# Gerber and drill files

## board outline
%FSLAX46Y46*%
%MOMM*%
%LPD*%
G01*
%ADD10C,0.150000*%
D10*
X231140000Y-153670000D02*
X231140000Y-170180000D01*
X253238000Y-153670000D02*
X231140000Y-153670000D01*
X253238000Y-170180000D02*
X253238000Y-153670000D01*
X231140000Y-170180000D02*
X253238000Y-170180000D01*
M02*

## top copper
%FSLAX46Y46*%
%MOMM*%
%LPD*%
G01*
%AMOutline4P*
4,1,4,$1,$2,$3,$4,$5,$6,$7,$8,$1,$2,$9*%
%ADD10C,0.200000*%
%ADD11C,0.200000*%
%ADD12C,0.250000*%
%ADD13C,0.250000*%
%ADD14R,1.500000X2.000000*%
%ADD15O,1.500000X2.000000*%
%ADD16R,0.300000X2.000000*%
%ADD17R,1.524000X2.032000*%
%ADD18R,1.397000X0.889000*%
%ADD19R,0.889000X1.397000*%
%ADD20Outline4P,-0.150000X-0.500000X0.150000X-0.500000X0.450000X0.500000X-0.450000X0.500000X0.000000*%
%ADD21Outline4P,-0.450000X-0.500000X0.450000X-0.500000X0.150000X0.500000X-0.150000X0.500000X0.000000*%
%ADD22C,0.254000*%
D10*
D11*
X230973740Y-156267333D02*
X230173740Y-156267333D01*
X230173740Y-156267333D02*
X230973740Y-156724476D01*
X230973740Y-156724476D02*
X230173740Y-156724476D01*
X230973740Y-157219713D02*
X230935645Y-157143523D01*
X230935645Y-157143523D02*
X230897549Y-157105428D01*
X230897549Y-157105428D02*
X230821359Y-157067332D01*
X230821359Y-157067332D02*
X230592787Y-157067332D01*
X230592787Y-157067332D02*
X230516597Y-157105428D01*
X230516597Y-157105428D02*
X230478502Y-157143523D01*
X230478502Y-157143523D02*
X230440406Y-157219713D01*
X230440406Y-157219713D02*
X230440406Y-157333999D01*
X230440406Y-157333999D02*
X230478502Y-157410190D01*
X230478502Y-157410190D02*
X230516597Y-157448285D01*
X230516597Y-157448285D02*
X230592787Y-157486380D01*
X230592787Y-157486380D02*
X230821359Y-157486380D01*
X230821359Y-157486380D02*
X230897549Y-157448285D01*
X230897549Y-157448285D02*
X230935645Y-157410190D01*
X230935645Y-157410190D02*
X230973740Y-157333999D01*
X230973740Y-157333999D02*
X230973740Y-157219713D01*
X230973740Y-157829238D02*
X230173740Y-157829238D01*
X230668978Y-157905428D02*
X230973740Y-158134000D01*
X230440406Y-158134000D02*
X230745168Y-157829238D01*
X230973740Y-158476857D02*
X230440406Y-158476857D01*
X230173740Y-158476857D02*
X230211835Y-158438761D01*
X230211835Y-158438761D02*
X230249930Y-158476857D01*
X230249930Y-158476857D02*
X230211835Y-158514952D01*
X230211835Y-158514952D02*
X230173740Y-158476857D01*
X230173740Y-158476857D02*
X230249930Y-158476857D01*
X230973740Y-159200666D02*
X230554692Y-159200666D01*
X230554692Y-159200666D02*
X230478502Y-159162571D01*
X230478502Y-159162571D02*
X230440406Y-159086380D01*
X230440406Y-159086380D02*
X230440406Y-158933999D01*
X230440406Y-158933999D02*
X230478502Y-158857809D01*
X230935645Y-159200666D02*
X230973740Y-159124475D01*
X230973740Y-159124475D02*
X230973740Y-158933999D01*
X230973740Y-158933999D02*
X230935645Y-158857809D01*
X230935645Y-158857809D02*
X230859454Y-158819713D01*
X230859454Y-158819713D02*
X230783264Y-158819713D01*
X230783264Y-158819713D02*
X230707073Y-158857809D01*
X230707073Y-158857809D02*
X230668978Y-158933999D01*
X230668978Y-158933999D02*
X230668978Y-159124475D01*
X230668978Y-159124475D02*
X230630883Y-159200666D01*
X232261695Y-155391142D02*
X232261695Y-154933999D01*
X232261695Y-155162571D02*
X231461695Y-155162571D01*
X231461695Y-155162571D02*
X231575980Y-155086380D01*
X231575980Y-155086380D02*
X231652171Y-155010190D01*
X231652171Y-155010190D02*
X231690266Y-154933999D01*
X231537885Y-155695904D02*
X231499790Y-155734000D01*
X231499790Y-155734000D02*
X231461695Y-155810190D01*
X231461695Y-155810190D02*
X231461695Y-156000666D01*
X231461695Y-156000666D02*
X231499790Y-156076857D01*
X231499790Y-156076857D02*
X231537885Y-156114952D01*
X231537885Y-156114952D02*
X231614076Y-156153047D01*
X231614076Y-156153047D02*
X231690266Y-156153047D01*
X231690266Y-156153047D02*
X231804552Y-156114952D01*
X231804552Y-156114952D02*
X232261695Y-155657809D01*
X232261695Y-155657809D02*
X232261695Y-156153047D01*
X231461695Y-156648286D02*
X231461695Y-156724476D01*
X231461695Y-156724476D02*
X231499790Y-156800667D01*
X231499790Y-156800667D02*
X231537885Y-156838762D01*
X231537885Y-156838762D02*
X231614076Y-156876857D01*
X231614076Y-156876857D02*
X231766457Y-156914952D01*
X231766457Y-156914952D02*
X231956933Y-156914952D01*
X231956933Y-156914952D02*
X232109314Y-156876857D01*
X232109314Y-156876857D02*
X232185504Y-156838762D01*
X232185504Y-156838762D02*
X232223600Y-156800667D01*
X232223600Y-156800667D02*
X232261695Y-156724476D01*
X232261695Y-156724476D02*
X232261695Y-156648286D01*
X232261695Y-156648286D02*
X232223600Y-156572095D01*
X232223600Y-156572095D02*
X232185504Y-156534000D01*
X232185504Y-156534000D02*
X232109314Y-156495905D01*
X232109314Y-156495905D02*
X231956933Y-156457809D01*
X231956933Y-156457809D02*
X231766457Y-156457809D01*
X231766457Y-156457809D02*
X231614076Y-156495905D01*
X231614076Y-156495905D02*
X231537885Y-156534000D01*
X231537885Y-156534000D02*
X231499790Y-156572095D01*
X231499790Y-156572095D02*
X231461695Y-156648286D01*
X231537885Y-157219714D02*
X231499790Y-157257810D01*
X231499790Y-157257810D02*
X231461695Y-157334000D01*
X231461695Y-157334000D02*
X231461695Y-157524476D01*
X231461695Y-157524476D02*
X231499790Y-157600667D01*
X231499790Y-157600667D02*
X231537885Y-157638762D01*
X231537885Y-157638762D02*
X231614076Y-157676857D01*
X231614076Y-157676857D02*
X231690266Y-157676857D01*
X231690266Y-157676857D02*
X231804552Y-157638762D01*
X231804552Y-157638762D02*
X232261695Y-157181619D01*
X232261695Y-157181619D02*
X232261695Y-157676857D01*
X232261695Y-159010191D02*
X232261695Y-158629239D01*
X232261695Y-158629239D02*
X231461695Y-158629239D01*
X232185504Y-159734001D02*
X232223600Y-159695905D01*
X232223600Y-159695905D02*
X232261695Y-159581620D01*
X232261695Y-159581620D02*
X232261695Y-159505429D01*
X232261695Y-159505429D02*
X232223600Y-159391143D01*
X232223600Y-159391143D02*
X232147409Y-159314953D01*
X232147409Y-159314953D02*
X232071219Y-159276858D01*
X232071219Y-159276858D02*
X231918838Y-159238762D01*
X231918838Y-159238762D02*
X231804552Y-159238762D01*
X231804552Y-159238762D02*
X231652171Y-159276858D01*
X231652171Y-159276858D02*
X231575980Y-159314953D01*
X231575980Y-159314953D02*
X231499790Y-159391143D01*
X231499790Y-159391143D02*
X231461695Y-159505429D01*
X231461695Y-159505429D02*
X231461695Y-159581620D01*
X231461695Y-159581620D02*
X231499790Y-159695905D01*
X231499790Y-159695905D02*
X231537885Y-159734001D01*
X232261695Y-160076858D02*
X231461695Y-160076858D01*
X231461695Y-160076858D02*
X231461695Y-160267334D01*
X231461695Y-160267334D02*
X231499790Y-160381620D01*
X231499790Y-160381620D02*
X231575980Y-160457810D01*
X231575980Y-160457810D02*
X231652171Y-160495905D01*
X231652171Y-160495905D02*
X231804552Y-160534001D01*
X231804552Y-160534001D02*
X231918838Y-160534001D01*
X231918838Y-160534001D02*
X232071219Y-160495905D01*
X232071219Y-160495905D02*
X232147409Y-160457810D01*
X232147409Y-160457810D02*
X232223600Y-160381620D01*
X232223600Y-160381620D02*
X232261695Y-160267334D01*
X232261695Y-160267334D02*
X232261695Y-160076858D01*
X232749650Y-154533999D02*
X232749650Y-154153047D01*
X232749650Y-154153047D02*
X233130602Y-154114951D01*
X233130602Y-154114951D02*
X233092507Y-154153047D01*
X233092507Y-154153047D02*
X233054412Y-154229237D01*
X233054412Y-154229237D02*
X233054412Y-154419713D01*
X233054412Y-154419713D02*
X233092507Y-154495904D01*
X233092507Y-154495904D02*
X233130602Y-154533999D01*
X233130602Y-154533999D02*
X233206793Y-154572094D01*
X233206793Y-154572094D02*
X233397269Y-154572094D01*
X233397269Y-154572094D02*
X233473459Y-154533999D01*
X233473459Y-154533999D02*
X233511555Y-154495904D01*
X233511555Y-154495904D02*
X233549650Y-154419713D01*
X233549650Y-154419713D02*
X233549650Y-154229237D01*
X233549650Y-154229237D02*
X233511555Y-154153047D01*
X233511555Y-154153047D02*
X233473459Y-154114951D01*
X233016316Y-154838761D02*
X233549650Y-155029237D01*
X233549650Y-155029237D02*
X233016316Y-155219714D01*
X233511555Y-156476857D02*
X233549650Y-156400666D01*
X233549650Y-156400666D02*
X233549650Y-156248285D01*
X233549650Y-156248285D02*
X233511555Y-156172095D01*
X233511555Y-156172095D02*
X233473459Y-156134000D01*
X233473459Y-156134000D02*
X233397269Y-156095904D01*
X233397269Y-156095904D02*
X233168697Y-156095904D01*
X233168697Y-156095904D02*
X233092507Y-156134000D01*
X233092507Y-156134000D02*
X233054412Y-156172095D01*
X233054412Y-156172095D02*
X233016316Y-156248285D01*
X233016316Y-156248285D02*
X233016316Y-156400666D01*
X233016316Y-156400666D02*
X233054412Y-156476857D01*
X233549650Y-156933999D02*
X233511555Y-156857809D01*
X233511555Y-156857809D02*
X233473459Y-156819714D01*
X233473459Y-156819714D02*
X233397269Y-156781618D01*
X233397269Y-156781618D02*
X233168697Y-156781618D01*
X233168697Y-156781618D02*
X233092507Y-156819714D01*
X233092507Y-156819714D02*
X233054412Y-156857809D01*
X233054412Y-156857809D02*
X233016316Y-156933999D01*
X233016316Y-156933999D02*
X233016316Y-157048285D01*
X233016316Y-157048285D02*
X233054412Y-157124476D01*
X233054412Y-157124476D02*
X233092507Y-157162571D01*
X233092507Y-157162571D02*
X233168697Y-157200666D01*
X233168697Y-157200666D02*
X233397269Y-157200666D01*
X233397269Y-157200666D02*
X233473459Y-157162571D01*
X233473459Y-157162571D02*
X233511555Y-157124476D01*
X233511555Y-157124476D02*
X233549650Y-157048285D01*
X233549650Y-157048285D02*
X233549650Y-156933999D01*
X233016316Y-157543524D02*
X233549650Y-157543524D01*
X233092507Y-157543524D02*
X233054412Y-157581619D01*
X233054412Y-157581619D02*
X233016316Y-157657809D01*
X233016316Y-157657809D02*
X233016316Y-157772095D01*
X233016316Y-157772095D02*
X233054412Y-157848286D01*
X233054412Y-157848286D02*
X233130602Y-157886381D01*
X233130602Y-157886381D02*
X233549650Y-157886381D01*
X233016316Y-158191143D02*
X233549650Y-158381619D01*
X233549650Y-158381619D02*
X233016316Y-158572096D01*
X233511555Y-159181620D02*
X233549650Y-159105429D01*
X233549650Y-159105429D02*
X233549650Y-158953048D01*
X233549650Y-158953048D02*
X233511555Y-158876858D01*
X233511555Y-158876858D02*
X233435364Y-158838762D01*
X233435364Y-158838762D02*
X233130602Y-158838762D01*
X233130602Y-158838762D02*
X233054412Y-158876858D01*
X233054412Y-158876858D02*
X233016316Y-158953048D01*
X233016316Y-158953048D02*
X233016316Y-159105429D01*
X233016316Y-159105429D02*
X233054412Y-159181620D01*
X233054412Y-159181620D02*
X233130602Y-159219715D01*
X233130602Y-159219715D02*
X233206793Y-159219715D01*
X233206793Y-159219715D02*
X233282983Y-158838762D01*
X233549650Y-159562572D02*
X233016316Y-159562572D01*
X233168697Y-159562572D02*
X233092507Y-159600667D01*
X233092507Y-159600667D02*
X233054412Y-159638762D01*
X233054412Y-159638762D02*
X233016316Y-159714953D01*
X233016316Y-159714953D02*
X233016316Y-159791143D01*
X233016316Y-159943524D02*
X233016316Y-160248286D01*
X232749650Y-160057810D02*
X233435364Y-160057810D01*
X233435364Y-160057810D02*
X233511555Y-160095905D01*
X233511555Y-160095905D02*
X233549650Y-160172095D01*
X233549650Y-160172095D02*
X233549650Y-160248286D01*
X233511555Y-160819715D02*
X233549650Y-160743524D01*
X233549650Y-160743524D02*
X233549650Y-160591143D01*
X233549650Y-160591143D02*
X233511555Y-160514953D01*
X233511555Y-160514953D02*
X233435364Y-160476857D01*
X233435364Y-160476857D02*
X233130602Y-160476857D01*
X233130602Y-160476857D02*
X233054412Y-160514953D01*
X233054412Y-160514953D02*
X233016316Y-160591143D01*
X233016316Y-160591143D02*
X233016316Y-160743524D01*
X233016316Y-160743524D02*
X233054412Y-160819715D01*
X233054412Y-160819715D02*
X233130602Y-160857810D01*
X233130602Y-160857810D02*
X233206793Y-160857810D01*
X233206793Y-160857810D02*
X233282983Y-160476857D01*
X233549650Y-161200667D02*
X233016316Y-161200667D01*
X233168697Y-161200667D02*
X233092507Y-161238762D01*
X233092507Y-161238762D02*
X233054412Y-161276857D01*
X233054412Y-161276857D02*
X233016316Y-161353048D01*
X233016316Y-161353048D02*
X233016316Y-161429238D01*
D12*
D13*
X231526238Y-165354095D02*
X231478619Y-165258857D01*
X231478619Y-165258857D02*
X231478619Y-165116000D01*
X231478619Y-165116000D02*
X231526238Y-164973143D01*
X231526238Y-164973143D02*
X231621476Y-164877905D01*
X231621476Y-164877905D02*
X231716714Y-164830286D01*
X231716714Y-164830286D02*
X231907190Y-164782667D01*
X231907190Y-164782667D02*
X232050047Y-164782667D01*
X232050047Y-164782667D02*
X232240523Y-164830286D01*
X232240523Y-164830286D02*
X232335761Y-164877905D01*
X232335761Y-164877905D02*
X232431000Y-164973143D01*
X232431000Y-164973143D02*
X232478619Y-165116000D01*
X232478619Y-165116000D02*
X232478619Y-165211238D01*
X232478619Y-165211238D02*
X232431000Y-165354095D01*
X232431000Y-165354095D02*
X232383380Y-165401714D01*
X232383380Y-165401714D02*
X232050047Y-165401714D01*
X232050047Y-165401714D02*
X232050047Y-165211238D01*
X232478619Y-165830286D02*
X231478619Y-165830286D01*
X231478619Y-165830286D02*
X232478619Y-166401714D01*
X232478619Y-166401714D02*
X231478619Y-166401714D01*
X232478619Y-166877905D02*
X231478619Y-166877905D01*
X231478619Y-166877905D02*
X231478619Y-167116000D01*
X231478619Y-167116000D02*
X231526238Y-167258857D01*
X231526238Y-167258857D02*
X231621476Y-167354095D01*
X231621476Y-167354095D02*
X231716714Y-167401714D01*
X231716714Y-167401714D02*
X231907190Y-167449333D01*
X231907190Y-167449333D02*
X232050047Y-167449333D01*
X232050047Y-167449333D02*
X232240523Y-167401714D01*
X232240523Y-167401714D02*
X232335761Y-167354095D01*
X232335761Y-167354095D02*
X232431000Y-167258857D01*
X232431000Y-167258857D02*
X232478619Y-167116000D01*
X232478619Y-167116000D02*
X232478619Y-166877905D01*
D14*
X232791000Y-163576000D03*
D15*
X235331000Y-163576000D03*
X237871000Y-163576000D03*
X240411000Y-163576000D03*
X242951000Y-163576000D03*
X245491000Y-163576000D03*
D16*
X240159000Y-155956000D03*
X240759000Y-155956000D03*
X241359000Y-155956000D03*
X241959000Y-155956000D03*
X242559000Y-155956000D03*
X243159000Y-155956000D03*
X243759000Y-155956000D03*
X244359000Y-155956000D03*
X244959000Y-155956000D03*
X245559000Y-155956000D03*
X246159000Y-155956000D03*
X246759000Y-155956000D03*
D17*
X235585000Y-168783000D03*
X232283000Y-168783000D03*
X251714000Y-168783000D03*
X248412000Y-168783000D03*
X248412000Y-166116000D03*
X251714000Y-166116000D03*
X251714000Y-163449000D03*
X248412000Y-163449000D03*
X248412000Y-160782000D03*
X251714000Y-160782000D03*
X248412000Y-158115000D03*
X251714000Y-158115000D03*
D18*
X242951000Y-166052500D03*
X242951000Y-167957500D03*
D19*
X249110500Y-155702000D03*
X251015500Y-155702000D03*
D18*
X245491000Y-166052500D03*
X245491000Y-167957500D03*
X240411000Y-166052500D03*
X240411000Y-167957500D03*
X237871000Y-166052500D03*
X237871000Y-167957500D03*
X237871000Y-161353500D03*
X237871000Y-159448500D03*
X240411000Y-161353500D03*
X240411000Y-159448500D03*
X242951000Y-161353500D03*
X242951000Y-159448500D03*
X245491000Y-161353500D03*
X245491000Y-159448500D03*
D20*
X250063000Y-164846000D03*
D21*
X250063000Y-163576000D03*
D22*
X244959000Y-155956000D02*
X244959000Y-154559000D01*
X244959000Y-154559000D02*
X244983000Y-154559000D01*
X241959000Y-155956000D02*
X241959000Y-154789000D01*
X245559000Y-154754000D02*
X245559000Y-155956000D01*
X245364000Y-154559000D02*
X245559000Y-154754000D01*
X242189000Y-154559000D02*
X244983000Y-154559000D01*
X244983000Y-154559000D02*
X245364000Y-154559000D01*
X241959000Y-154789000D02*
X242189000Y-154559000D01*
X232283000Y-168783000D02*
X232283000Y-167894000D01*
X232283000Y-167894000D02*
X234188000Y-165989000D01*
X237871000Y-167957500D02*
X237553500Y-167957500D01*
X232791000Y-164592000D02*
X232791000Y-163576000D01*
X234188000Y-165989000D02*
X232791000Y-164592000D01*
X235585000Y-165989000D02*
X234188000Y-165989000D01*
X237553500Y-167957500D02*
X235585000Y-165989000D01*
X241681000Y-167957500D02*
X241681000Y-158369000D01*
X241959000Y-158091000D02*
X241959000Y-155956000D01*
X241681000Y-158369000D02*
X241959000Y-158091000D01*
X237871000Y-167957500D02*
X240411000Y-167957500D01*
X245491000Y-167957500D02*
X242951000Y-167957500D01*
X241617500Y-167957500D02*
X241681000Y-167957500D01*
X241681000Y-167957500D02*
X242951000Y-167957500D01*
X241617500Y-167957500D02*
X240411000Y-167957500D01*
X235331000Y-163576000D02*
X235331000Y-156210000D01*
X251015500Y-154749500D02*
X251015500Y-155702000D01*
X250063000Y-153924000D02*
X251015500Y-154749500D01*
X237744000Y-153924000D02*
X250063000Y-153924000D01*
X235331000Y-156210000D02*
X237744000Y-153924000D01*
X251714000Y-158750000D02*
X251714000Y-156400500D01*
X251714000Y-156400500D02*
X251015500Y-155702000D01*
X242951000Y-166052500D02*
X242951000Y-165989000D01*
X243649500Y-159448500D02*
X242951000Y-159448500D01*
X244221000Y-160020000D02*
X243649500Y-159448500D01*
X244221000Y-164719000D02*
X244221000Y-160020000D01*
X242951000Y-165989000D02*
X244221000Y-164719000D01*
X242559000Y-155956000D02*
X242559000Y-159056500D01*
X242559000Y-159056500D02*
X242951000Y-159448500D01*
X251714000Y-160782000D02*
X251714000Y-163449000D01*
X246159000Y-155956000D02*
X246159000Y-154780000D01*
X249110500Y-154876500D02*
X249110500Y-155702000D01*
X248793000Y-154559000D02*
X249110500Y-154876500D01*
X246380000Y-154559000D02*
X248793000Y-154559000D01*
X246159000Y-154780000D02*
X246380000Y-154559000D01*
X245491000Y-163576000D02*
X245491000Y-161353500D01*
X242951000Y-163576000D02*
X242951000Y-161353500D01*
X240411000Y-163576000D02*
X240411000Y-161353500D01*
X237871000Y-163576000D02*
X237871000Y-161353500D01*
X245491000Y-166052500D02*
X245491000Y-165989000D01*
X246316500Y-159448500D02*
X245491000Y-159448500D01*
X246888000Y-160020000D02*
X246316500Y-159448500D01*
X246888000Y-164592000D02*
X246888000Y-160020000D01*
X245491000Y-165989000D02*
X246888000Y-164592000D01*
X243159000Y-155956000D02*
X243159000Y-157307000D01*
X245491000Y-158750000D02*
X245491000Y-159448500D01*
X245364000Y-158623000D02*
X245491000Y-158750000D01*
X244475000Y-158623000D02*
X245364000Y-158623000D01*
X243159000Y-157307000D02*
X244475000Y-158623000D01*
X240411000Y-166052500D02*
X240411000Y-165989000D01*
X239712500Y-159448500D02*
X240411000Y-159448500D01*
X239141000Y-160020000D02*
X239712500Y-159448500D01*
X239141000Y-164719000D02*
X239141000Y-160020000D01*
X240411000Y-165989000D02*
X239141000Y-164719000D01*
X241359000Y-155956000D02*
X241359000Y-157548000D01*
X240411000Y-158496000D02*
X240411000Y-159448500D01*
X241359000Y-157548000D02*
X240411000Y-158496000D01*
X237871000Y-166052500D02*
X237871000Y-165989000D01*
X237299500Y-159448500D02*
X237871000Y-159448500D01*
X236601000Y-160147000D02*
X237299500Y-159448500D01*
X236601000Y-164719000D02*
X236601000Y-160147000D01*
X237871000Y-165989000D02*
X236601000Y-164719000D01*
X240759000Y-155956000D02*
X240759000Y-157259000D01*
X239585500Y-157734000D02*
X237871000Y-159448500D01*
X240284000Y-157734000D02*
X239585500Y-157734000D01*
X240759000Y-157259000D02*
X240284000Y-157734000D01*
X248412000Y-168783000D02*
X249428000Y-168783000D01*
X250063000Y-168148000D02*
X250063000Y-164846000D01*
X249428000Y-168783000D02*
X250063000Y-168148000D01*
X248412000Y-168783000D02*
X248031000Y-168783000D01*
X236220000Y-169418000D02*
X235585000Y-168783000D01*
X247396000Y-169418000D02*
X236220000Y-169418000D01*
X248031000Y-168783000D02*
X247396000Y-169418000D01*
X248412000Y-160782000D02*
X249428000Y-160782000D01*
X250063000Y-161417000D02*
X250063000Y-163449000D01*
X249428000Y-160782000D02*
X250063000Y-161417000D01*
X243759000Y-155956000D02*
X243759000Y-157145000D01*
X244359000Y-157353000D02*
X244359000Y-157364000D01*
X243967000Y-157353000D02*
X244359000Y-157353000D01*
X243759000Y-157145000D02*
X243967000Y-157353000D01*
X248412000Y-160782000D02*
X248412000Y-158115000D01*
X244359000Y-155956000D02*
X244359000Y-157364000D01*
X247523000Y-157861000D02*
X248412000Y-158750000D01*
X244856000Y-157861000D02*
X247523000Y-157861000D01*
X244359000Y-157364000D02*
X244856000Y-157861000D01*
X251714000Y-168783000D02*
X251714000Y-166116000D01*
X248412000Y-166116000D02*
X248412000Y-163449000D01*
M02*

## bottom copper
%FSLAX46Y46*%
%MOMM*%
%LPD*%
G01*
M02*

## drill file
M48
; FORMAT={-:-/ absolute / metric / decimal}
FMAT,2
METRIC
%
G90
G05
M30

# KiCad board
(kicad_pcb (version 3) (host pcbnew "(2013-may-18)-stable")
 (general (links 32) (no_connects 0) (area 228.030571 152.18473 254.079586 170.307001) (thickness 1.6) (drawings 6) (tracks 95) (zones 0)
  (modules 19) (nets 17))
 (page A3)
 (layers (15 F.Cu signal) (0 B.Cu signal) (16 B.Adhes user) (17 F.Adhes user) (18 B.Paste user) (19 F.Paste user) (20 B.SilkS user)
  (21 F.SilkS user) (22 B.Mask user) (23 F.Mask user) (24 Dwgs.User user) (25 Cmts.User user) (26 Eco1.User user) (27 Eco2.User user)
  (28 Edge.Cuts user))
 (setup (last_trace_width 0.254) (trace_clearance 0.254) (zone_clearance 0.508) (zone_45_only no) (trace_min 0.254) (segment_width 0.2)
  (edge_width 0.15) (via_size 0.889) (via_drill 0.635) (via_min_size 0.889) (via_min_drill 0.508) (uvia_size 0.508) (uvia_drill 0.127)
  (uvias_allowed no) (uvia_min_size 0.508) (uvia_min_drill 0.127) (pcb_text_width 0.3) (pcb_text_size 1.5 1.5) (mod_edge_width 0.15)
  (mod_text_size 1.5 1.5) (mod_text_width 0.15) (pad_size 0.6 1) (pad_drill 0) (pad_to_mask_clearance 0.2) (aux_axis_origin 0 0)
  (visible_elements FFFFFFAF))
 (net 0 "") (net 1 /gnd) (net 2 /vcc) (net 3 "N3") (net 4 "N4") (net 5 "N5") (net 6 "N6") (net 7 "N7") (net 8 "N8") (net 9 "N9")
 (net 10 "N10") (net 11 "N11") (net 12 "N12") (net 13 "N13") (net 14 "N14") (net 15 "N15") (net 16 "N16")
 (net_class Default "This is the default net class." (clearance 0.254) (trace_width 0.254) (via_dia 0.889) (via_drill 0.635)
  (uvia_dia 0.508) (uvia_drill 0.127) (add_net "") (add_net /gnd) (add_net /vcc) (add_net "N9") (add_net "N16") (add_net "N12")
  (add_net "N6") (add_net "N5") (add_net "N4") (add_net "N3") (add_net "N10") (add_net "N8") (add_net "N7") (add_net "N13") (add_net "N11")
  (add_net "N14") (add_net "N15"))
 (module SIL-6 (layer F.Cu) (at 239.141 163.576)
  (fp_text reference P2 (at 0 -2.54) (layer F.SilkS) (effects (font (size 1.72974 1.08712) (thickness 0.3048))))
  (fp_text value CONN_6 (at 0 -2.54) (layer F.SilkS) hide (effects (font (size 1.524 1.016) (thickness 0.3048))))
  (pad 1 connect rect (at -6.35 0) (size 1.5 2) (layers F.Cu F.Mask) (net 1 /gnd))
  (pad 2 connect oval (at -3.81 0) (size 1.5 2) (layers F.Cu F.Mask) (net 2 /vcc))
  (pad 3 connect oval (at -1.27 0) (size 1.5 2) (layers F.Cu F.Mask) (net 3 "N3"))
  (pad 4 connect oval (at 1.27 0) (size 1.5 2) (layers F.Cu F.Mask) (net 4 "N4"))
  (pad 5 connect oval (at 3.81 0) (size 1.5 2) (layers F.Cu F.Mask) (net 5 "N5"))
  (pad 6 connect oval (at 6.35 0) (size 1.5 2) (layers F.Cu F.Mask) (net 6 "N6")))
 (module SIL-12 (layer F.Cu) (at 243.459 155.956)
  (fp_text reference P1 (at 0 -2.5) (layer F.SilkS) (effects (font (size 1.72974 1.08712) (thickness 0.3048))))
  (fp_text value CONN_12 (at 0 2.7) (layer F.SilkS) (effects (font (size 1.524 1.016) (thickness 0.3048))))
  (pad 1 connect rect (at -3.3 0) (size 0.3 2) (layers F.Cu F.Mask) (clearance 0.15))
  (pad 2 connect rect (at -2.7 0) (size 0.3 2) (layers F.Cu F.Mask) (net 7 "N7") (clearance 0.15))
  (pad 3 connect rect (at -2.1 0) (size 0.3 2) (layers F.Cu F.Mask) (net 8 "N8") (clearance 0.15))
  (pad 4 connect rect (at -1.5 0) (size 0.3 2) (layers F.Cu F.Mask) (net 1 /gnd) (clearance 0.15))
  (pad 5 connect rect (at -0.9 0) (size 0.3 2) (layers F.Cu F.Mask) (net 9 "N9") (clearance 0.15))
  (pad 6 connect rect (at -0.3 0) (size 0.3 2) (layers F.Cu F.Mask) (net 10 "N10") (clearance 0.15))
  (pad 7 connect rect (at 0.3 0) (size 0.3 2) (layers F.Cu F.Mask) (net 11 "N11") (clearance 0.15))
  (pad 8 connect rect (at 0.9 0) (size 0.3 2) (layers F.Cu F.Mask) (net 11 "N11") (clearance 0.15))
  (pad 9 connect rect (at 1.5 0) (size 0.3 2) (layers F.Cu F.Mask) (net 1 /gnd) (clearance 0.15))
  (pad 10 connect rect (at 2.1 0) (size 0.3 2) (layers F.Cu F.Mask) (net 1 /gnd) (clearance 0.15))
  (pad 11 connect rect (at 2.7 0) (size 0.3 2) (layers F.Cu F.Mask) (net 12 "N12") (clearance 0.15))
  (pad 12 connect rect (at 3.3 0) (size 0.3 2) (layers F.Cu F.Mask) (clearance 0.15)))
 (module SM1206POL (layer F.Cu) (at 233.934 168.783 180)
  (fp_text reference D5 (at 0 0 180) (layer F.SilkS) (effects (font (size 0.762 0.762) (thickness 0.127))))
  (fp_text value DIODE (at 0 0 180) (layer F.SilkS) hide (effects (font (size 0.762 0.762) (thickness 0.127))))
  (pad 1 smd rect (at -1.651 0 180) (size 1.524 2.032) (layers F.Cu F.Paste F.Mask) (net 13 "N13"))
  (pad 2 smd rect (at 1.651 0 180) (size 1.524 2.032) (layers F.Cu F.Paste F.Mask) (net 1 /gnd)))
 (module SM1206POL (layer F.Cu) (at 250.063 168.783 180)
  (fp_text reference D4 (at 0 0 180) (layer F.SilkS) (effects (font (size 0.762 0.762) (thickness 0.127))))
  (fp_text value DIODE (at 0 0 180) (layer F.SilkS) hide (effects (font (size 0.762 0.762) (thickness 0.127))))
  (pad 1 smd rect (at -1.651 0 180) (size 1.524 2.032) (layers F.Cu F.Paste F.Mask) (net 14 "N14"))
  (pad 2 smd rect (at 1.651 0 180) (size 1.524 2.032) (layers F.Cu F.Paste F.Mask) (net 13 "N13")))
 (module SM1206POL (layer F.Cu) (at 250.063 166.116)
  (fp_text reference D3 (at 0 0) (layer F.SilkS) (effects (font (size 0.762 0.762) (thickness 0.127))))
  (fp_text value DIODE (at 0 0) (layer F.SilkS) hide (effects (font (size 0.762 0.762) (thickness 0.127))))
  (pad 1 smd rect (at -1.651 0) (size 1.524 2.032) (layers F.Cu F.Paste F.Mask) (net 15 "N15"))
  (pad 2 smd rect (at 1.651 0) (size 1.524 2.032) (layers F.Cu F.Paste F.Mask) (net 14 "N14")))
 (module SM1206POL (layer F.Cu) (at 250.063 163.449 180)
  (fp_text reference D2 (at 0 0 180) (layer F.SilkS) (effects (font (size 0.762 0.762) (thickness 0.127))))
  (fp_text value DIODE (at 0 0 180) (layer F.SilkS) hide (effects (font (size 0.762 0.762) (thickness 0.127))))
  (pad 1 smd rect (at -1.651 0 180) (size 1.524 2.032) (layers F.Cu F.Paste F.Mask) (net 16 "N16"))
  (pad 2 smd rect (at 1.651 0 180) (size 1.524 2.032) (layers F.Cu F.Paste F.Mask) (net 15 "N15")))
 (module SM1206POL (layer F.Cu) (at 250.063 160.782)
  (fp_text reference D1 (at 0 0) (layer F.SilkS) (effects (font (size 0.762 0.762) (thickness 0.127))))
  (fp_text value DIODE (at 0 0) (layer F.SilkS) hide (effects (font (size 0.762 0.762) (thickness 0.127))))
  (pad 1 smd rect (at -1.651 0) (size 1.524 2.032) (layers F.Cu F.Paste F.Mask) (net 11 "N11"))
  (pad 2 smd rect (at 1.651 0) (size 1.524 2.032) (layers F.Cu F.Paste F.Mask) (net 16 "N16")))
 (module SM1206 (layer F.Cu) (at 250.063 158.115)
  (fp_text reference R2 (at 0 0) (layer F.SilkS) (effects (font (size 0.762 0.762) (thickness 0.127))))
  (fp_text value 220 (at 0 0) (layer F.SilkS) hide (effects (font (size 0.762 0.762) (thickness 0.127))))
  (pad 1 smd rect (at -1.651 0) (size 1.524 2.032) (layers F.Cu F.Paste F.Mask) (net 11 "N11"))
  (pad 2 smd rect (at 1.651 0) (size 1.524 2.032) (layers F.Cu F.Paste F.Mask) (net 2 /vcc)))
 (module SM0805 (layer F.Cu) (at 242.951 167.005 270)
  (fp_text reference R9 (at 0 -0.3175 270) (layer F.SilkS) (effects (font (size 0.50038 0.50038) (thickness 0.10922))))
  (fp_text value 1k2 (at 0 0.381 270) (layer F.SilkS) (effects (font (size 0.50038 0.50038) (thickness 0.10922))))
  (pad 1 smd rect (at -0.9525 0 270) (size 0.889 1.397) (layers F.Cu F.Paste F.Mask) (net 9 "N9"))
  (pad 2 smd rect (at 0.9525 0 270) (size 0.889 1.397) (layers F.Cu F.Paste F.Mask) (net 1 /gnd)))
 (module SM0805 (layer F.Cu) (at 250.063 155.702)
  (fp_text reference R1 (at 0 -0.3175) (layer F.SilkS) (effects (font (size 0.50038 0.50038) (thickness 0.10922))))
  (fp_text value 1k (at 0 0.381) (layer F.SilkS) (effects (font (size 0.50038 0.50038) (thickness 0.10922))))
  (pad 1 smd rect (at -0.9525 0) (size 0.889 1.397) (layers F.Cu F.Paste F.Mask) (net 12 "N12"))
  (pad 2 smd rect (at 0.9525 0) (size 0.889 1.397) (layers F.Cu F.Paste F.Mask) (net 2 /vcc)))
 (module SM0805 (layer F.Cu) (at 245.491 167.005 270)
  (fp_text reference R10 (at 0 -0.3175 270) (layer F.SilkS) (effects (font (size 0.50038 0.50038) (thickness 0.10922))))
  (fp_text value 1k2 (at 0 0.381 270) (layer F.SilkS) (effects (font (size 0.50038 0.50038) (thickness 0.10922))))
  (pad 1 smd rect (at -0.9525 0 270) (size 0.889 1.397) (layers F.Cu F.Paste F.Mask) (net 10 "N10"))
  (pad 2 smd rect (at 0.9525 0 270) (size 0.889 1.397) (layers F.Cu F.Paste F.Mask) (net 1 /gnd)))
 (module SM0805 (layer F.Cu) (at 240.411 167.005 270)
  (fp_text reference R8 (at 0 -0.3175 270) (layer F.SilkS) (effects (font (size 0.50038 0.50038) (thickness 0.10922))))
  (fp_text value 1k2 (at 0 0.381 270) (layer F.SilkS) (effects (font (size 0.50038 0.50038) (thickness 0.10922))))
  (pad 1 smd rect (at -0.9525 0 270) (size 0.889 1.397) (layers F.Cu F.Paste F.Mask) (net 8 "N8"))
  (pad 2 smd rect (at 0.9525 0 270) (size 0.889 1.397) (layers F.Cu F.Paste F.Mask) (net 1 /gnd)))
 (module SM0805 (layer F.Cu) (at 237.871 167.005 270)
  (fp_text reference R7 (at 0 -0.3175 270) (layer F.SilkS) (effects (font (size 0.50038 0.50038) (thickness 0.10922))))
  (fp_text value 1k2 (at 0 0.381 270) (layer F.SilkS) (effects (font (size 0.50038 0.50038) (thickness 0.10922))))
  (pad 1 smd rect (at -0.9525 0 270) (size 0.889 1.397) (layers F.Cu F.Paste F.Mask) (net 7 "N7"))
  (pad 2 smd rect (at 0.9525 0 270) (size 0.889 1.397) (layers F.Cu F.Paste F.Mask) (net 1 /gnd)))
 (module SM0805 (layer F.Cu) (at 237.871 160.401 90)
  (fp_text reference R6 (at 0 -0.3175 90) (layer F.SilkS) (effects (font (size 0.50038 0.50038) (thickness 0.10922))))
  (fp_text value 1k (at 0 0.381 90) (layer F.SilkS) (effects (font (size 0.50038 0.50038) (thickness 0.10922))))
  (pad 1 smd rect (at -0.9525 0 90) (size 0.889 1.397) (layers F.Cu F.Paste F.Mask) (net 3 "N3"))
  (pad 2 smd rect (at 0.9525 0 90) (size 0.889 1.397) (layers F.Cu F.Paste F.Mask) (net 7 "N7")))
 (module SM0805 (layer F.Cu) (at 240.411 160.401 90)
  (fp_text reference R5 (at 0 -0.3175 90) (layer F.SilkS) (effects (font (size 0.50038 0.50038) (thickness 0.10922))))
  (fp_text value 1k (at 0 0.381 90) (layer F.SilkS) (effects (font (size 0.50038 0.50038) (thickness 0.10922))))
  (pad 1 smd rect (at -0.9525 0 90) (size 0.889 1.397) (layers F.Cu F.Paste F.Mask) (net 4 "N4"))
  (pad 2 smd rect (at 0.9525 0 90) (size 0.889 1.397) (layers F.Cu F.Paste F.Mask) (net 8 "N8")))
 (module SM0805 (layer F.Cu) (at 242.951 160.401 90)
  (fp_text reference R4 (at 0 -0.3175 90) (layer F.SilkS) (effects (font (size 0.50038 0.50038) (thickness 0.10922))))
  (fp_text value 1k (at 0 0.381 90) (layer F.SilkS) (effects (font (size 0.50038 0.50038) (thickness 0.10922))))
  (pad 1 smd rect (at -0.9525 0 90) (size 0.889 1.397) (layers F.Cu F.Paste F.Mask) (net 5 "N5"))
  (pad 2 smd rect (at 0.9525 0 90) (size 0.889 1.397) (layers F.Cu F.Paste F.Mask) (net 9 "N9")))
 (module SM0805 (layer F.Cu) (at 245.491 160.401 90)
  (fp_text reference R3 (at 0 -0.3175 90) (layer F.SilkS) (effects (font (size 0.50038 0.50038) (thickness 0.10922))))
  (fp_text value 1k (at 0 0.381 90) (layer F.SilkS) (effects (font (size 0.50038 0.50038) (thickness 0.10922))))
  (pad 1 smd rect (at -0.9525 0 90) (size 0.889 1.397) (layers F.Cu F.Paste F.Mask) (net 6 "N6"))
  (pad 2 smd rect (at 0.9525 0 90) (size 0.889 1.397) (layers F.Cu F.Paste F.Mask) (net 10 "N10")))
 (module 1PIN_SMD (layer F.Cu) (at 250.063 164.846)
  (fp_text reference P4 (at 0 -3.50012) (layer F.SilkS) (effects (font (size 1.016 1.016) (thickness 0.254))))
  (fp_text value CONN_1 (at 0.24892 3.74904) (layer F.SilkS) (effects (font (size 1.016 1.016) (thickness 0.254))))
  (pad 1 smd trapezoid (at 0 0) (size 0.6 1) (rect_delta 0 -0.3) (layers F.Cu F.Paste F.SilkS F.Mask) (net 13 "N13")))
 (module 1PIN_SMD (layer F.Cu) (at 250.063 163.576)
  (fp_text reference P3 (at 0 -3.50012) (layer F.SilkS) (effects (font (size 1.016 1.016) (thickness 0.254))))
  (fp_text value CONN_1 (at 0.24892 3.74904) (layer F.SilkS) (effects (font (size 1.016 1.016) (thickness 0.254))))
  (pad 1 smd trapezoid (at 0 0) (size 0.6 1) (rect_delta 0 0.3) (layers F.Cu F.Paste F.SilkS F.Mask) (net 11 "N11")))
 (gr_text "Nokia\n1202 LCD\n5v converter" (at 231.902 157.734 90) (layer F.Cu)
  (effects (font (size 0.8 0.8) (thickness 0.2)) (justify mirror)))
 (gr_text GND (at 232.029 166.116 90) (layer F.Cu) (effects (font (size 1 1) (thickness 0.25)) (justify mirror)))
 (gr_line (start 231.14 153.67) (end 231.14 170.18) (angle 90) (layer Edge.Cuts) (width 0.15))
 (gr_line (start 253.238 153.67) (end 231.14 153.67) (angle 90) (layer Edge.Cuts) (width 0.15))
 (gr_line (start 253.238 170.18) (end 253.238 153.67) (angle 90) (layer Edge.Cuts) (width 0.15))
 (gr_line (start 231.14 170.18) (end 253.238 170.18) (angle 90) (layer Edge.Cuts) (width 0.15))
 (segment (start 244.959 155.956) (end 244.959 154.559) (width 0.254) (layer F.Cu) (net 1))
 (segment (start 244.959 154.559) (end 244.983 154.559) (width 0.254) (layer F.Cu) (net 1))
 (segment (start 241.959 155.956) (end 241.959 154.789) (width 0.254) (layer F.Cu) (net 1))
 (segment (start 245.559 154.754) (end 245.559 155.956) (width 0.254) (layer F.Cu) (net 1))
 (segment (start 245.364 154.559) (end 245.559 154.754) (width 0.254) (layer F.Cu) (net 1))
 (segment (start 242.189 154.559) (end 244.983 154.559) (width 0.254) (layer F.Cu) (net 1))
 (segment (start 244.983 154.559) (end 245.364 154.559) (width 0.254) (layer F.Cu) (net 1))
 (segment (start 241.959 154.789) (end 242.189 154.559) (width 0.254) (layer F.Cu) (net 1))
 (segment (start 232.283 168.783) (end 232.283 167.894) (width 0.254) (layer F.Cu) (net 1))
 (segment (start 232.283 167.894) (end 234.188 165.989) (width 0.254) (layer F.Cu) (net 1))
 (segment (start 237.871 167.9575) (end 237.5535 167.9575) (width 0.254) (layer F.Cu) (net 1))
 (segment (start 232.791 164.592) (end 232.791 163.576) (width 0.254) (layer F.Cu) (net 1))
 (segment (start 234.188 165.989) (end 232.791 164.592) (width 0.254) (layer F.Cu) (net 1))
 (segment (start 235.585 165.989) (end 234.188 165.989) (width 0.254) (layer F.Cu) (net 1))
 (segment (start 237.5535 167.9575) (end 235.585 165.989) (width 0.254) (layer F.Cu) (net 1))
 (segment (start 241.681 167.9575) (end 241.681 158.369) (width 0.254) (layer F.Cu) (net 1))
 (segment (start 241.959 158.091) (end 241.959 155.956) (width 0.254) (layer F.Cu) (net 1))
 (segment (start 241.681 158.369) (end 241.959 158.091) (width 0.254) (layer F.Cu) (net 1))
 (segment (start 237.871 167.9575) (end 240.411 167.9575) (width 0.254) (layer F.Cu) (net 1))
 (segment (start 245.491 167.9575) (end 242.951 167.9575) (width 0.254) (layer F.Cu) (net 1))
 (segment (start 241.6175 167.9575) (end 241.681 167.9575) (width 0.254) (layer F.Cu) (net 1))
 (segment (start 241.681 167.9575) (end 242.951 167.9575) (width 0.254) (layer F.Cu) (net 1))
 (segment (start 241.6175 167.9575) (end 240.411 167.9575) (width 0.254) (layer F.Cu) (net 1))
 (segment (start 235.331 163.576) (end 235.331 156.21) (width 0.254) (layer F.Cu) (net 2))
 (segment (start 251.0155 154.7495) (end 251.0155 155.702) (width 0.254) (layer F.Cu) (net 2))
 (segment (start 250.063 153.924) (end 251.0155 154.7495) (width 0.254) (layer F.Cu) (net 2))
 (segment (start 237.744 153.924) (end 250.063 153.924) (width 0.254) (layer F.Cu) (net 2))
 (segment (start 235.331 156.21) (end 237.744 153.924) (width 0.254) (layer F.Cu) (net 2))
 (segment (start 251.714 158.75) (end 251.714 156.4005) (width 0.254) (layer F.Cu) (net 2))
 (segment (start 251.714 156.4005) (end 251.0155 155.702) (width 0.254) (layer F.Cu) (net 2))
 (segment (start 242.951 166.0525) (end 242.951 165.989) (width 0.254) (layer F.Cu) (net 9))
 (segment (start 243.6495 159.4485) (end 242.951 159.4485) (width 0.254) (layer F.Cu) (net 9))
 (segment (start 244.221 160.02) (end 243.6495 159.4485) (width 0.254) (layer F.Cu) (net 9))
 (segment (start 244.221 164.719) (end 244.221 160.02) (width 0.254) (layer F.Cu) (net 9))
 (segment (start 242.951 165.989) (end 244.221 164.719) (width 0.254) (layer F.Cu) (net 9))
 (segment (start 242.559 155.956) (end 242.559 159.0565) (width 0.254) (layer F.Cu) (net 9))
 (segment (start 242.559 159.0565) (end 242.951 159.4485) (width 0.254) (layer F.Cu) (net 9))
 (segment (start 251.714 160.782) (end 251.714 163.449) (width 0.254) (layer F.Cu) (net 16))
 (segment (start 246.159 155.956) (end 246.159 154.78) (width 0.254) (layer F.Cu) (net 12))
 (segment (start 249.1105 154.8765) (end 249.1105 155.702) (width 0.254) (layer F.Cu) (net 12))
 (segment (start 248.793 154.559) (end 249.1105 154.8765) (width 0.254) (layer F.Cu) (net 12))
 (segment (start 246.38 154.559) (end 248.793 154.559) (width 0.254) (layer F.Cu) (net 12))
 (segment (start 246.159 154.78) (end 246.38 154.559) (width 0.254) (layer F.Cu) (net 12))
 (segment (start 245.491 163.576) (end 245.491 161.3535) (width 0.254) (layer F.Cu) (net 6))
 (segment (start 242.951 163.576) (end 242.951 161.3535) (width 0.254) (layer F.Cu) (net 5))
 (segment (start 240.411 163.576) (end 240.411 161.3535) (width 0.254) (layer F.Cu) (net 4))
 (segment (start 237.871 163.576) (end 237.871 161.3535) (width 0.254) (layer F.Cu) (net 3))
 (segment (start 245.491 166.0525) (end 245.491 165.989) (width 0.254) (layer F.Cu) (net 10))
 (segment (start 246.3165 159.4485) (end 245.491 159.4485) (width 0.254) (layer F.Cu) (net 10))
 (segment (start 246.888 160.02) (end 246.3165 159.4485) (width 0.254) (layer F.Cu) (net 10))
 (segment (start 246.888 164.592) (end 246.888 160.02) (width 0.254) (layer F.Cu) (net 10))
 (segment (start 245.491 165.989) (end 246.888 164.592) (width 0.254) (layer F.Cu) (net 10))
 (segment (start 243.159 155.956) (end 243.159 157.307) (width 0.254) (layer F.Cu) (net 10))
 (segment (start 245.491 158.75) (end 245.491 159.4485) (width 0.254) (layer F.Cu) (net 10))
 (segment (start 245.364 158.623) (end 245.491 158.75) (width 0.254) (layer F.Cu) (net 10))
 (segment (start 244.475 158.623) (end 245.364 158.623) (width 0.254) (layer F.Cu) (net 10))
 (segment (start 243.159 157.307) (end 244.475 158.623) (width 0.254) (layer F.Cu) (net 10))
 (segment (start 240.411 166.0525) (end 240.411 165.989) (width 0.254) (layer F.Cu) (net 8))
 (segment (start 239.7125 159.4485) (end 240.411 159.4485) (width 0.254) (layer F.Cu) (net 8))
 (segment (start 239.141 160.02) (end 239.7125 159.4485) (width 0.254) (layer F.Cu) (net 8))
 (segment (start 239.141 164.719) (end 239.141 160.02) (width 0.254) (layer F.Cu) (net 8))
 (segment (start 240.411 165.989) (end 239.141 164.719) (width 0.254) (layer F.Cu) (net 8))
 (segment (start 241.359 155.956) (end 241.359 157.548) (width 0.254) (layer F.Cu) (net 8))
 (segment (start 240.411 158.496) (end 240.411 159.4485) (width 0.254) (layer F.Cu) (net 8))
 (segment (start 241.359 157.548) (end 240.411 158.496) (width 0.254) (layer F.Cu) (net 8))
 (segment (start 237.871 166.0525) (end 237.871 165.989) (width 0.254) (layer F.Cu) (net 7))
 (segment (start 237.2995 159.4485) (end 237.871 159.4485) (width 0.254) (layer F.Cu) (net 7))
 (segment (start 236.601 160.147) (end 237.2995 159.4485) (width 0.254) (layer F.Cu) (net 7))
 (segment (start 236.601 164.719) (end 236.601 160.147) (width 0.254) (layer F.Cu) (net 7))
 (segment (start 237.871 165.989) (end 236.601 164.719) (width 0.254) (layer F.Cu) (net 7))
 (segment (start 240.759 155.956) (end 240.759 157.259) (width 0.254) (layer F.Cu) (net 7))
 (segment (start 239.5855 157.734) (end 237.871 159.4485) (width 0.254) (layer F.Cu) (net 7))
 (segment (start 240.284 157.734) (end 239.5855 157.734) (width 0.254) (layer F.Cu) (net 7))
 (segment (start 240.759 157.259) (end 240.284 157.734) (width 0.254) (layer F.Cu) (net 7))
 (segment (start 248.412 168.783) (end 249.428 168.783) (width 0.254) (layer F.Cu) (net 13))
 (segment (start 250.063 168.148) (end 250.063 164.846) (width 0.254) (layer F.Cu) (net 13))
 (segment (start 249.428 168.783) (end 250.063 168.148) (width 0.254) (layer F.Cu) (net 13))
 (segment (start 248.412 168.783) (end 248.031 168.783) (width 0.254) (layer F.Cu) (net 13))
 (segment (start 236.22 169.418) (end 235.585 168.783) (width 0.254) (layer F.Cu) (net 13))
 (segment (start 247.396 169.418) (end 236.22 169.418) (width 0.254) (layer F.Cu) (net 13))
 (segment (start 248.031 168.783) (end 247.396 169.418) (width 0.254) (layer F.Cu) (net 13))
 (segment (start 248.412 160.782) (end 249.428 160.782) (width 0.254) (layer F.Cu) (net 11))
 (segment (start 250.063 161.417) (end 250.063 163.449) (width 0.254) (layer F.Cu) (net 11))
 (segment (start 249.428 160.782) (end 250.063 161.417) (width 0.254) (layer F.Cu) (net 11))
 (segment (start 243.759 155.956) (end 243.759 157.145) (width 0.254) (layer F.Cu) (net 11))
 (segment (start 244.359 157.353) (end 244.359 157.364) (width 0.254) (layer F.Cu) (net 11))
 (segment (start 243.967 157.353) (end 244.359 157.353) (width 0.254) (layer F.Cu) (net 11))
 (segment (start 243.759 157.145) (end 243.967 157.353) (width 0.254) (layer F.Cu) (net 11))
 (segment (start 248.412 160.782) (end 248.412 158.115) (width 0.254) (layer F.Cu) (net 11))
 (segment (start 244.359 155.956) (end 244.359 157.364) (width 0.254) (layer F.Cu) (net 11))
 (segment (start 247.523 157.861) (end 248.412 158.75) (width 0.254) (layer F.Cu) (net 11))
 (segment (start 244.856 157.861) (end 247.523 157.861) (width 0.254) (layer F.Cu) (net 11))
 (segment (start 244.359 157.364) (end 244.856 157.861) (width 0.254) (layer F.Cu) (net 11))
 (segment (start 251.714 168.783) (end 251.714 166.116) (width 0.254) (layer F.Cu) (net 14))
 (segment (start 248.412 166.116) (end 248.412 163.449) (width 0.254) (layer F.Cu) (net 15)))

